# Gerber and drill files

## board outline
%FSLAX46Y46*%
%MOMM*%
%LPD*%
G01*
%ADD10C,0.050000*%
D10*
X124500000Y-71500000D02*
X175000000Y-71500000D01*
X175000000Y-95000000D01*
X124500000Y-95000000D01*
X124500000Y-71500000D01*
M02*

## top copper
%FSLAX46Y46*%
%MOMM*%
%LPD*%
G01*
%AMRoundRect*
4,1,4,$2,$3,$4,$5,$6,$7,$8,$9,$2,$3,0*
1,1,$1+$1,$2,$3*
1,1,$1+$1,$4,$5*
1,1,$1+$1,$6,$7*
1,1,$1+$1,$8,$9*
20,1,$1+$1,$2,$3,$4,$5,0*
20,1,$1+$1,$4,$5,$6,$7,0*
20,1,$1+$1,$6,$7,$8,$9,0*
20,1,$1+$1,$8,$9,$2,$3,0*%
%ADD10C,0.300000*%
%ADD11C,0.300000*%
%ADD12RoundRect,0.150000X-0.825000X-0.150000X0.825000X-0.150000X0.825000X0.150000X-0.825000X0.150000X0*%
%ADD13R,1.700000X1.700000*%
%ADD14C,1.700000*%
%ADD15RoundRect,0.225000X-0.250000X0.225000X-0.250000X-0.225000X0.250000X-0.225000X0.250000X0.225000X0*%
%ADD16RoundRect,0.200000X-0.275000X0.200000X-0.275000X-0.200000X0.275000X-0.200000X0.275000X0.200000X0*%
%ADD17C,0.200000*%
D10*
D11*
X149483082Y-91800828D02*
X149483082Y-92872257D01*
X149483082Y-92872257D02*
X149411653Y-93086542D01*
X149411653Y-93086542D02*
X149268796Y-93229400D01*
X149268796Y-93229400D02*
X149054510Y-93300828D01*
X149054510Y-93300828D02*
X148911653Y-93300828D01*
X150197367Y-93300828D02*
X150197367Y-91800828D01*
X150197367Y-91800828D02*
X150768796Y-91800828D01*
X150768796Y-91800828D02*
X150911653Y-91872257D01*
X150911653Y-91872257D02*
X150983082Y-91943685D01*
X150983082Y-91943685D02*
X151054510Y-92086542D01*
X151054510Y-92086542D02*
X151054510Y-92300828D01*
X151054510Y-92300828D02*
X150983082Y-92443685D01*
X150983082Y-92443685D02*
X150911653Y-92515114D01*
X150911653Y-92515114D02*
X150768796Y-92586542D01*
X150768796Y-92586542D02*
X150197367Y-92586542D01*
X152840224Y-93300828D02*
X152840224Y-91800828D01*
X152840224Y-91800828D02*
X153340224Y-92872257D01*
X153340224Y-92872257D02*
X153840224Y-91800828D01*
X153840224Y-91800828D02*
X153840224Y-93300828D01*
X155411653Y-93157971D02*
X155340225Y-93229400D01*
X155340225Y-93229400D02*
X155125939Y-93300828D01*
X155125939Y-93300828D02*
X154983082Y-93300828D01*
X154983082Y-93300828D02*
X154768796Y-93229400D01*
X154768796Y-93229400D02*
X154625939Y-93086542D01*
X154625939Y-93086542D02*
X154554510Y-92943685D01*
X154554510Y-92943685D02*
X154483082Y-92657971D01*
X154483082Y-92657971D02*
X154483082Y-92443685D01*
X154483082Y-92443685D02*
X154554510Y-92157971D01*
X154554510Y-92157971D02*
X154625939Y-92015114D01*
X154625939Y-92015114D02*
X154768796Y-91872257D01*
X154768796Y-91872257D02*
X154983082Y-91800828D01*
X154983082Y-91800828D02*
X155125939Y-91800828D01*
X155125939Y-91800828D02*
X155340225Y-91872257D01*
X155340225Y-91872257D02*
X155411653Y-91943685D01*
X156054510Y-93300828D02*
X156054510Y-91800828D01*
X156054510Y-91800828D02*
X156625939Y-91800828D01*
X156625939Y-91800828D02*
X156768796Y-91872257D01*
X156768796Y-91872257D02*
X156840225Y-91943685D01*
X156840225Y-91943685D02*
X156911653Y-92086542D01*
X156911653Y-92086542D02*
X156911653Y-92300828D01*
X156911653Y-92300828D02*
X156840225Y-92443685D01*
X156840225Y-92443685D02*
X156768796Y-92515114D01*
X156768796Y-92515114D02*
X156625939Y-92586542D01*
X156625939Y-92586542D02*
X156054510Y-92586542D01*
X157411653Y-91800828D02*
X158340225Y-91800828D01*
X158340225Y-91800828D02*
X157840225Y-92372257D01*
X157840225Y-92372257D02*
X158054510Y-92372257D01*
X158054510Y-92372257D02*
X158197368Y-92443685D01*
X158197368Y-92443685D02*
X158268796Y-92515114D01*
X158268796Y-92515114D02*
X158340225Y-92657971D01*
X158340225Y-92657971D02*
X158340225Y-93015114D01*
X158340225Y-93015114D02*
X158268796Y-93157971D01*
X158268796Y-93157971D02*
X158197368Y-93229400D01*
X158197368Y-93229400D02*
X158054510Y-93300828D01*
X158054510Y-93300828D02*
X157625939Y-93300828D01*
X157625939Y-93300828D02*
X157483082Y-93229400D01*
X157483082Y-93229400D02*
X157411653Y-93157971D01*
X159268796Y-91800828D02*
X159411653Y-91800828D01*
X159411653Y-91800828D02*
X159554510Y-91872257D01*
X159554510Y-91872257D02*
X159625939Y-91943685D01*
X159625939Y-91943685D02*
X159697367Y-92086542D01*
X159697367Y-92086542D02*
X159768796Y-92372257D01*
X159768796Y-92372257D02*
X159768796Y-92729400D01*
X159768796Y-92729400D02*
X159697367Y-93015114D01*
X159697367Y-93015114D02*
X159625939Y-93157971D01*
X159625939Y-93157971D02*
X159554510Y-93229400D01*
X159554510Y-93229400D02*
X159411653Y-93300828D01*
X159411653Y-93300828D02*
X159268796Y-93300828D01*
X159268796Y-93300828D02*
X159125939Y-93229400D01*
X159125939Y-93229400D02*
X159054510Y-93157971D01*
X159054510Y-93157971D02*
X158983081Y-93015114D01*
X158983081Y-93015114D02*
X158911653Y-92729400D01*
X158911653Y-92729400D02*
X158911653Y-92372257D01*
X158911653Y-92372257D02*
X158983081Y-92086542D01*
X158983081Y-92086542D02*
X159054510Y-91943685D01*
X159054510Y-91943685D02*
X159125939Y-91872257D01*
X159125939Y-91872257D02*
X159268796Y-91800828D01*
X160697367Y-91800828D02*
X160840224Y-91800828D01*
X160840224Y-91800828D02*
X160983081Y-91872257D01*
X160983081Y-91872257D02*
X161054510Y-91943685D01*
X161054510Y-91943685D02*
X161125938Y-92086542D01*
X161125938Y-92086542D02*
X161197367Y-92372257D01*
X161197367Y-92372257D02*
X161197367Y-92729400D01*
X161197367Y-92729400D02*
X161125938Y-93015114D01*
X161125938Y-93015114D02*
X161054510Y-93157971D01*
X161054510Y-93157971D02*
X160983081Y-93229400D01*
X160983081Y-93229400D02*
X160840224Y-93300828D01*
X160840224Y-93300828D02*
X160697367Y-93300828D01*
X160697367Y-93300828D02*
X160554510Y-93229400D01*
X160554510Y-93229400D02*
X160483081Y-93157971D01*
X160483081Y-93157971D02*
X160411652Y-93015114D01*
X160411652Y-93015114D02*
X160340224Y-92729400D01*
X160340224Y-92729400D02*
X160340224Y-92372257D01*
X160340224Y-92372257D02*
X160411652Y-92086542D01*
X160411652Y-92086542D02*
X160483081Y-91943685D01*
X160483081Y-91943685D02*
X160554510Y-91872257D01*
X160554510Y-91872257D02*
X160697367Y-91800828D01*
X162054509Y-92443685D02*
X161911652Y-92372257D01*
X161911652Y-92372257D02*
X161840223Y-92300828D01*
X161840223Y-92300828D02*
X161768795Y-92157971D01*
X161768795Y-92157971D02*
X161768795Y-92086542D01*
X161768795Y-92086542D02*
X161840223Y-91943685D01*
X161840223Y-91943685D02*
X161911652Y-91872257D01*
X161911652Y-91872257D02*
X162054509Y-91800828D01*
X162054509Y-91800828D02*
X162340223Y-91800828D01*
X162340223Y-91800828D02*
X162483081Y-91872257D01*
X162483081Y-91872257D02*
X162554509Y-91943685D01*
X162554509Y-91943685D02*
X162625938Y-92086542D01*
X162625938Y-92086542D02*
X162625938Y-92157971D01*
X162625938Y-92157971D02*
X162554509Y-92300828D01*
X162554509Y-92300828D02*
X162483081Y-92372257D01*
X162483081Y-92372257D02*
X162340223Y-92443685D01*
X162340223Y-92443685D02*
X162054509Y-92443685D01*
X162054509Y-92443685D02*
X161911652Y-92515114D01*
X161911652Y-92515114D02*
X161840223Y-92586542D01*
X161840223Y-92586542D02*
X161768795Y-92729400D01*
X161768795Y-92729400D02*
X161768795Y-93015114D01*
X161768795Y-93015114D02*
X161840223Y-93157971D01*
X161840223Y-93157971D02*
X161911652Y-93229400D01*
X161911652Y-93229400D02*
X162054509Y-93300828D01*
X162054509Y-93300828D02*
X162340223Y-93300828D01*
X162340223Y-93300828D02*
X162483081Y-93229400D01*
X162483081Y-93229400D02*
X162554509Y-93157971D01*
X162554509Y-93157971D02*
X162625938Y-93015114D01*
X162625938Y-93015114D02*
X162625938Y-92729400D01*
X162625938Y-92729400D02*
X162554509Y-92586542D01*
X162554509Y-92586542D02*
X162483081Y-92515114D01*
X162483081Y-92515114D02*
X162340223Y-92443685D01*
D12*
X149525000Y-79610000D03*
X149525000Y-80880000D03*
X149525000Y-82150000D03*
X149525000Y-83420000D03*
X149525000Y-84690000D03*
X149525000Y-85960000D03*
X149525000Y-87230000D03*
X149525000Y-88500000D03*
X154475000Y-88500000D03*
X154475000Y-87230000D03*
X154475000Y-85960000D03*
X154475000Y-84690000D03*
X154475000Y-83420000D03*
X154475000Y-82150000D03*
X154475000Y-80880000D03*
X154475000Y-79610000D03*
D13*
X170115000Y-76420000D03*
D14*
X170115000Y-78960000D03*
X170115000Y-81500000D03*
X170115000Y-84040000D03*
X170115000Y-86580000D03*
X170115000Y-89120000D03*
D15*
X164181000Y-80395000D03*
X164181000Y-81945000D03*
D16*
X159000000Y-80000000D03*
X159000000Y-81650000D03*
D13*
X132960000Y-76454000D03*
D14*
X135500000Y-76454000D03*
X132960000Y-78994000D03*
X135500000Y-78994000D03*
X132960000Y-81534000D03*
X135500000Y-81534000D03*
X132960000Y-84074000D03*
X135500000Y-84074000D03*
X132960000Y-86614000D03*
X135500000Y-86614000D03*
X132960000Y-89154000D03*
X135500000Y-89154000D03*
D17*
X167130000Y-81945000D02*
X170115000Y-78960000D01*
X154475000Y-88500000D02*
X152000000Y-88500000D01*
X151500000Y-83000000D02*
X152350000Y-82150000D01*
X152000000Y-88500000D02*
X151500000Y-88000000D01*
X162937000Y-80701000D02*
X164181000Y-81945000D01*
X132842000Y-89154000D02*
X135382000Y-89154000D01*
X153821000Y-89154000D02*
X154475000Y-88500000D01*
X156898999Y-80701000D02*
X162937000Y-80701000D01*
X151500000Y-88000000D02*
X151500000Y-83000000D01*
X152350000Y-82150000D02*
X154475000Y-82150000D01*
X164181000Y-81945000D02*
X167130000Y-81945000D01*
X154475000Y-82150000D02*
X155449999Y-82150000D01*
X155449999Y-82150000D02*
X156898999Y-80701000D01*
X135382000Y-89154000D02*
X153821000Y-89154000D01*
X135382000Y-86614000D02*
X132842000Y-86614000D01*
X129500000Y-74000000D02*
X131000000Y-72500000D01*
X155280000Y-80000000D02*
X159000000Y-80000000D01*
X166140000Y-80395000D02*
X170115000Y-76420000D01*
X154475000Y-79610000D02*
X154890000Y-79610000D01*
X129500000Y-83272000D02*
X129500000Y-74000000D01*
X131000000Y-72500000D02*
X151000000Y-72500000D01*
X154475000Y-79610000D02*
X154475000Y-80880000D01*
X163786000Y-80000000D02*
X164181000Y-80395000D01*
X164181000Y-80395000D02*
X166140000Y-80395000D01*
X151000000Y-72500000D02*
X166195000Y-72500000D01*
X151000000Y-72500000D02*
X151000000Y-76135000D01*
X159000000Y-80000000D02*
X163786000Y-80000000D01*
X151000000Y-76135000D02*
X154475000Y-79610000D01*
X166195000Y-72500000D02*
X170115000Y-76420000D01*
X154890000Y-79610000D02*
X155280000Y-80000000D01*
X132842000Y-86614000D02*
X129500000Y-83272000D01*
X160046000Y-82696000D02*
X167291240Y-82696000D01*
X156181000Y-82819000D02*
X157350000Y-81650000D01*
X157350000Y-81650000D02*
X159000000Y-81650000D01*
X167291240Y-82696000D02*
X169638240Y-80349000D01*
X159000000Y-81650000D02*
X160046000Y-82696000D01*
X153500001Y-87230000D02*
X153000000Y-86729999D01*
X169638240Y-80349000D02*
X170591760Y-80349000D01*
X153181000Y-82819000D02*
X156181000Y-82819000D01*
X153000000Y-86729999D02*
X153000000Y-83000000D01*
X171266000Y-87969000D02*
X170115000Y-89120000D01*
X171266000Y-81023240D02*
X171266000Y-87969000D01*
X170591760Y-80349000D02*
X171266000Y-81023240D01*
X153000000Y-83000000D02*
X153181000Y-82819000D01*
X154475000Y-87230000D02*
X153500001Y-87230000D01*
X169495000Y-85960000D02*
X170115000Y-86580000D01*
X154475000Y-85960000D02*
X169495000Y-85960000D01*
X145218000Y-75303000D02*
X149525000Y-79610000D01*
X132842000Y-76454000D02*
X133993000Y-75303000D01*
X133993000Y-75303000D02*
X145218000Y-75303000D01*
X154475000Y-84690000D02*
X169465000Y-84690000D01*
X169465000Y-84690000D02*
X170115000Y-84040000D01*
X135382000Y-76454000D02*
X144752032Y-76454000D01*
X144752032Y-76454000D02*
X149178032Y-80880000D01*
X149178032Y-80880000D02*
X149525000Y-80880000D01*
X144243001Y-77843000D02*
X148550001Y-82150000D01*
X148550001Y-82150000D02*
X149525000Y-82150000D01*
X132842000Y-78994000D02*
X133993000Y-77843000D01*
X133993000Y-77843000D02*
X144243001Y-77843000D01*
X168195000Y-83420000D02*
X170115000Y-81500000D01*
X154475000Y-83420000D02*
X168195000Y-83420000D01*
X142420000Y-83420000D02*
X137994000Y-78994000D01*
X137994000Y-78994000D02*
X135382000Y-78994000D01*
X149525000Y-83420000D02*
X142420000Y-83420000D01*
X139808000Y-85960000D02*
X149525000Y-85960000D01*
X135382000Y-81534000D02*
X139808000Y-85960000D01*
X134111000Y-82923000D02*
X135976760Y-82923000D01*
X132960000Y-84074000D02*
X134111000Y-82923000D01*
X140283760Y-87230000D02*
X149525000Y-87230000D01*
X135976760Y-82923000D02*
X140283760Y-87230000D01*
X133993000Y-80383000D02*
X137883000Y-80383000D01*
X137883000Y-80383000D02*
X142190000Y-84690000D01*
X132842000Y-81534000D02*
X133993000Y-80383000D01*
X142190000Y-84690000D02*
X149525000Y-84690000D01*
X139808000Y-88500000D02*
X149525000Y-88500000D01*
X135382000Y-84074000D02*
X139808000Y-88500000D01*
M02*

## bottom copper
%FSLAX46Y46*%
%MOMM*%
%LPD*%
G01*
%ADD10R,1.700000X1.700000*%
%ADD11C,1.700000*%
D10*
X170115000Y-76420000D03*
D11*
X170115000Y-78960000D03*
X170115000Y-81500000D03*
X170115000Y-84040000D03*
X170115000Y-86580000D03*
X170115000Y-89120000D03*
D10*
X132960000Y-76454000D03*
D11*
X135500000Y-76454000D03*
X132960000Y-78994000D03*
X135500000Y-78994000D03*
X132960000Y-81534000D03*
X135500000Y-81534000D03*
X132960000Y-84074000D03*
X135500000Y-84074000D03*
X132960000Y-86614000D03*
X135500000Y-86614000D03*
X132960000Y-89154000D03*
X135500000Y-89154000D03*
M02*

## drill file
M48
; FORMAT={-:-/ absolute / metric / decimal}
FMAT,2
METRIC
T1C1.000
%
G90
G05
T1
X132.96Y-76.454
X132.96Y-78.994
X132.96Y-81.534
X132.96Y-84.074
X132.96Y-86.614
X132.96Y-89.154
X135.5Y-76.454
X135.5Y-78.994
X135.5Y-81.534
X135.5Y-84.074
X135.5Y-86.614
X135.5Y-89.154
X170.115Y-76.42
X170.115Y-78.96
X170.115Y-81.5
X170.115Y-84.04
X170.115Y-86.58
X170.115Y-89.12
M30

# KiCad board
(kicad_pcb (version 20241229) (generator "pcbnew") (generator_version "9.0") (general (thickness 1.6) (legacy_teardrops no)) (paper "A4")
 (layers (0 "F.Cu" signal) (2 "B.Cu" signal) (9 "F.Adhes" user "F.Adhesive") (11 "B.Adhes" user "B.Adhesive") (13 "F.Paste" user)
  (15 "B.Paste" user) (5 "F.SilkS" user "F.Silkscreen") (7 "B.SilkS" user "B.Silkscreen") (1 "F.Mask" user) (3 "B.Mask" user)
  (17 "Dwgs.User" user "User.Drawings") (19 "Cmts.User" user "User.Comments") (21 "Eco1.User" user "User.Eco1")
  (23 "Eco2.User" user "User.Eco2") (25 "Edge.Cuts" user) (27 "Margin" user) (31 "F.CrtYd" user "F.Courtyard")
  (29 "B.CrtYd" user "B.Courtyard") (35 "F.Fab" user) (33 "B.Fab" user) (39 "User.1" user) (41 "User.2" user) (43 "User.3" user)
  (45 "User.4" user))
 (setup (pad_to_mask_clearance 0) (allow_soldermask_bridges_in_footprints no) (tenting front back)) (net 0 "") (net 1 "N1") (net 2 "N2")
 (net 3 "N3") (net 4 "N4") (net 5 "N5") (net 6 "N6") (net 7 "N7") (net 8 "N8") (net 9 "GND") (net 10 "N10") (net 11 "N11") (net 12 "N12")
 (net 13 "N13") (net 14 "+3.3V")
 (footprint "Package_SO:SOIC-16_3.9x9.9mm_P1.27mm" (layer "F.Cu") (at 152 84.055)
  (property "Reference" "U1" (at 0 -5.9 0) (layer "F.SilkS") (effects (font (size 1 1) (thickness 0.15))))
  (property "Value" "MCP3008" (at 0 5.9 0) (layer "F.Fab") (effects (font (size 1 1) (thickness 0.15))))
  (pad "1" smd roundrect (at -2.475 -4.445) (size 1.95 0.6) (layers "F.Cu" "F.Mask" "F.Paste") (roundrect_rratio 0.25) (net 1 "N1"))
  (pad "2" smd roundrect (at -2.475 -3.175) (size 1.95 0.6) (layers "F.Cu" "F.Mask" "F.Paste") (roundrect_rratio 0.25) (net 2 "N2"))
  (pad "3" smd roundrect (at -2.475 -1.905) (size 1.95 0.6) (layers "F.Cu" "F.Mask" "F.Paste") (roundrect_rratio 0.25) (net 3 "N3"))
  (pad "4" smd roundrect (at -2.475 -0.635) (size 1.95 0.6) (layers "F.Cu" "F.Mask" "F.Paste") (roundrect_rratio 0.25) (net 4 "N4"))
  (pad "5" smd roundrect (at -2.475 0.635) (size 1.95 0.6) (layers "F.Cu" "F.Mask" "F.Paste") (roundrect_rratio 0.25) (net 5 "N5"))
  (pad "6" smd roundrect (at -2.475 1.905) (size 1.95 0.6) (layers "F.Cu" "F.Mask" "F.Paste") (roundrect_rratio 0.25) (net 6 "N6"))
  (pad "7" smd roundrect (at -2.475 3.175) (size 1.95 0.6) (layers "F.Cu" "F.Mask" "F.Paste") (roundrect_rratio 0.25) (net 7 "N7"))
  (pad "8" smd roundrect (at -2.475 4.445) (size 1.95 0.6) (layers "F.Cu" "F.Mask" "F.Paste") (roundrect_rratio 0.25) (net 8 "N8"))
  (pad "9" smd roundrect (at 2.475 4.445) (size 1.95 0.6) (layers "F.Cu" "F.Mask" "F.Paste") (roundrect_rratio 0.25) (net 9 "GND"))
  (pad "10" smd roundrect (at 2.475 3.175) (size 1.95 0.6) (layers "F.Cu" "F.Mask" "F.Paste") (roundrect_rratio 0.25) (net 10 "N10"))
  (pad "11" smd roundrect (at 2.475 1.905) (size 1.95 0.6) (layers "F.Cu" "F.Mask" "F.Paste") (roundrect_rratio 0.25) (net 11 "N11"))
  (pad "12" smd roundrect (at 2.475 0.635) (size 1.95 0.6) (layers "F.Cu" "F.Mask" "F.Paste") (roundrect_rratio 0.25) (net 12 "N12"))
  (pad "13" smd roundrect (at 2.475 -0.635) (size 1.95 0.6) (layers "F.Cu" "F.Mask" "F.Paste") (roundrect_rratio 0.25) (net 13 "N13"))
  (pad "14" smd roundrect (at 2.475 -1.905) (size 1.95 0.6) (layers "F.Cu" "F.Mask" "F.Paste") (roundrect_rratio 0.25) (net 9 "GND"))
  (pad "15" smd roundrect (at 2.475 -3.175) (size 1.95 0.6) (layers "F.Cu" "F.Mask" "F.Paste") (roundrect_rratio 0.25) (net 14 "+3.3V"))
  (pad "16" smd roundrect (at 2.475 -4.445) (size 1.95 0.6) (layers "F.Cu" "F.Mask" "F.Paste") (roundrect_rratio 0.25) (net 14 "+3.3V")))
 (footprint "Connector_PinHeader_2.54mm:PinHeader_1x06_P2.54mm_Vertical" (layer "F.Cu") (at 170.115 76.42)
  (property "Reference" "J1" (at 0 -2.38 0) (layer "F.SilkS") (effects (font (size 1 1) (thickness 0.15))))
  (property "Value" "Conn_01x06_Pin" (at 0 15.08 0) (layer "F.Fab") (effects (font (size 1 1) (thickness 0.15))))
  (pad "1" thru_hole rect (at 0 0) (size 1.7 1.7) (drill 1) (layers "*.Cu" "*.Mask") (remove_unused_layers no) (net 14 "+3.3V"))
  (pad "2" thru_hole circle (at 0 2.54) (size 1.7 1.7) (drill 1) (layers "*.Cu" "*.Mask") (remove_unused_layers no) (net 9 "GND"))
  (pad "3" thru_hole circle (at 0 5.08) (size 1.7 1.7) (drill 1) (layers "*.Cu" "*.Mask") (remove_unused_layers no) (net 13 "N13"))
  (pad "4" thru_hole circle (at 0 7.62) (size 1.7 1.7) (drill 1) (layers "*.Cu" "*.Mask") (remove_unused_layers no) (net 12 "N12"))
  (pad "5" thru_hole circle (at 0 10.16) (size 1.7 1.7) (drill 1) (layers "*.Cu" "*.Mask") (remove_unused_layers no) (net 11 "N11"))
  (pad "6" thru_hole circle (at 0 12.7) (size 1.7 1.7) (drill 1) (layers "*.Cu" "*.Mask") (remove_unused_layers no) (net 10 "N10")))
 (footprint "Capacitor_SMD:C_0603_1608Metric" (layer "F.Cu") (at 164.181 81.17 -90)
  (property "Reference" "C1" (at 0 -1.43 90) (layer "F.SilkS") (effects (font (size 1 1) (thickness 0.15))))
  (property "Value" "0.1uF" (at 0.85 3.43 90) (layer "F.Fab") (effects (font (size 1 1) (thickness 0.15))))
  (pad "1" smd roundrect (at -0.775 0 270) (size 0.9 0.95) (layers "F.Cu" "F.Mask" "F.Paste") (roundrect_rratio 0.25) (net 14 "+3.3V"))
  (pad "2" smd roundrect (at 0.775 0 270) (size 0.9 0.95) (layers "F.Cu" "F.Mask" "F.Paste") (roundrect_rratio 0.25) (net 9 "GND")))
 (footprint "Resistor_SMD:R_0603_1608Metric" (layer "F.Cu") (at 159 80.825 -90)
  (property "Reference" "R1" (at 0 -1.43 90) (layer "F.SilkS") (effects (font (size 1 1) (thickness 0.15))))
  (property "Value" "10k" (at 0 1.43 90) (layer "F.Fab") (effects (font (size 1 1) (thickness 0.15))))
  (pad "1" smd roundrect (at -0.825 0 270) (size 0.8 0.95) (layers "F.Cu" "F.Mask" "F.Paste") (roundrect_rratio 0.25) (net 14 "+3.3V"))
  (pad "2" smd roundrect (at 0.825 0 270) (size 0.8 0.95) (layers "F.Cu" "F.Mask" "F.Paste") (roundrect_rratio 0.25) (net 10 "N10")))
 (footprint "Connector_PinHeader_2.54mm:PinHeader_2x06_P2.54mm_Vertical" (layer "F.Cu") (at 132.96 76.454)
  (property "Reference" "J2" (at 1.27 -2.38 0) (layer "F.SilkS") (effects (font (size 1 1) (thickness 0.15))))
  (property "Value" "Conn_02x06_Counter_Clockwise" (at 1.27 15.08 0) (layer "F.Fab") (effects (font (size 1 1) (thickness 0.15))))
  (pad "1" thru_hole rect (at 0 0) (size 1.7 1.7) (drill 1) (layers "*.Cu" "*.Mask") (remove_unused_layers no) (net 1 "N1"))
  (pad "2" thru_hole circle (at 2.54 0) (size 1.7 1.7) (drill 1) (layers "*.Cu" "*.Mask") (remove_unused_layers no) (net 2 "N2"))
  (pad "3" thru_hole circle (at 0 2.54) (size 1.7 1.7) (drill 1) (layers "*.Cu" "*.Mask") (remove_unused_layers no) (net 3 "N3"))
  (pad "4" thru_hole circle (at 2.54 2.54) (size 1.7 1.7) (drill 1) (layers "*.Cu" "*.Mask") (remove_unused_layers no) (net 4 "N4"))
  (pad "5" thru_hole circle (at 0 5.08) (size 1.7 1.7) (drill 1) (layers "*.Cu" "*.Mask") (remove_unused_layers no) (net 5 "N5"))
  (pad "6" thru_hole circle (at 2.54 5.08) (size 1.7 1.7) (drill 1) (layers "*.Cu" "*.Mask") (remove_unused_layers no) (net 6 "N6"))
  (pad "7" thru_hole circle (at 0 7.62) (size 1.7 1.7) (drill 1) (layers "*.Cu" "*.Mask") (remove_unused_layers no) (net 7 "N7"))
  (pad "8" thru_hole circle (at 2.54 7.62) (size 1.7 1.7) (drill 1) (layers "*.Cu" "*.Mask") (remove_unused_layers no) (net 8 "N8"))
  (pad "9" thru_hole circle (at 0 10.16) (size 1.7 1.7) (drill 1) (layers "*.Cu" "*.Mask") (remove_unused_layers no) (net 14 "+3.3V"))
  (pad "10" thru_hole circle (at 2.54 10.16) (size 1.7 1.7) (drill 1) (layers "*.Cu" "*.Mask") (remove_unused_layers no) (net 14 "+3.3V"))
  (pad "11" thru_hole circle (at 0 12.7) (size 1.7 1.7) (drill 1) (layers "*.Cu" "*.Mask") (remove_unused_layers no) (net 9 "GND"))
  (pad "12" thru_hole circle (at 2.54 12.7) (size 1.7 1.7) (drill 1) (layers "*.Cu" "*.Mask") (remove_unused_layers no) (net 9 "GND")))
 (gr_rect (start 124.5 71.5) (end 175 95) (stroke (width 0.05) (type solid)) (fill no) (layer "Edge.Cuts"))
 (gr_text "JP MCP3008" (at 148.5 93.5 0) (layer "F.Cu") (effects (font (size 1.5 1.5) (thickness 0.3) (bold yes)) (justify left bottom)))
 (segment (start 167.13 81.945) (end 170.115 78.96) (width 0.2) (layer "F.Cu") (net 9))
 (segment (start 154.475 88.5) (end 152 88.5) (width 0.2) (layer "F.Cu") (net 9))
 (segment (start 151.5 83) (end 152.35 82.15) (width 0.2) (layer "F.Cu") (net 9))
 (segment (start 152 88.5) (end 151.5 88) (width 0.2) (layer "F.Cu") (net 9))
 (segment (start 162.937 80.701) (end 164.181 81.945) (width 0.2) (layer "F.Cu") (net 9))
 (segment (start 132.842 89.154) (end 135.382 89.154) (width 0.2) (layer "F.Cu") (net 9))
 (segment (start 153.821 89.154) (end 154.475 88.5) (width 0.2) (layer "F.Cu") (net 9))
 (segment (start 156.898999 80.701) (end 162.937 80.701) (width 0.2) (layer "F.Cu") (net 9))
 (segment (start 151.5 88) (end 151.5 83) (width 0.2) (layer "F.Cu") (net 9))
 (segment (start 152.35 82.15) (end 154.475 82.15) (width 0.2) (layer "F.Cu") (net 9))
 (segment (start 164.181 81.945) (end 167.13 81.945) (width 0.2) (layer "F.Cu") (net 9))
 (segment (start 154.475 82.15) (end 155.449999 82.15) (width 0.2) (layer "F.Cu") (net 9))
 (segment (start 155.449999 82.15) (end 156.898999 80.701) (width 0.2) (layer "F.Cu") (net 9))
 (segment (start 135.382 89.154) (end 153.821 89.154) (width 0.2) (layer "F.Cu") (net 9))
 (segment (start 135.382 86.614) (end 132.842 86.614) (width 0.2) (layer "F.Cu") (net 14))
 (segment (start 129.5 74) (end 131 72.5) (width 0.2) (layer "F.Cu") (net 14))
 (segment (start 155.28 80) (end 159 80) (width 0.2) (layer "F.Cu") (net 14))
 (segment (start 166.14 80.395) (end 170.115 76.42) (width 0.2) (layer "F.Cu") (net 14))
 (segment (start 154.475 79.61) (end 154.89 79.61) (width 0.2) (layer "F.Cu") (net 14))
 (segment (start 129.5 83.272) (end 129.5 74) (width 0.2) (layer "F.Cu") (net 14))
 (segment (start 131 72.5) (end 151 72.5) (width 0.2) (layer "F.Cu") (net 14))
 (segment (start 154.475 79.61) (end 154.475 80.88) (width 0.2) (layer "F.Cu") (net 14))
 (segment (start 163.786 80) (end 164.181 80.395) (width 0.2) (layer "F.Cu") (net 14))
 (segment (start 164.181 80.395) (end 166.14 80.395) (width 0.2) (layer "F.Cu") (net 14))
 (segment (start 151 72.5) (end 166.195 72.5) (width 0.2) (layer "F.Cu") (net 14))
 (segment (start 151 72.5) (end 151 76.135) (width 0.2) (layer "F.Cu") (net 14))
 (segment (start 159 80) (end 163.786 80) (width 0.2) (layer "F.Cu") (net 14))
 (segment (start 151 76.135) (end 154.475 79.61) (width 0.2) (layer "F.Cu") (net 14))
 (segment (start 166.195 72.5) (end 170.115 76.42) (width 0.2) (layer "F.Cu") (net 14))
 (segment (start 154.89 79.61) (end 155.28 80) (width 0.2) (layer "F.Cu") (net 14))
 (segment (start 132.842 86.614) (end 129.5 83.272) (width 0.2) (layer "F.Cu") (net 14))
 (segment (start 160.046 82.696) (end 167.29124 82.696) (width 0.2) (layer "F.Cu") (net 10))
 (segment (start 156.181 82.819) (end 157.35 81.65) (width 0.2) (layer "F.Cu") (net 10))
 (segment (start 157.35 81.65) (end 159 81.65) (width 0.2) (layer "F.Cu") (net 10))
 (segment (start 167.29124 82.696) (end 169.63824 80.349) (width 0.2) (layer "F.Cu") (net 10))
 (segment (start 159 81.65) (end 160.046 82.696) (width 0.2) (layer "F.Cu") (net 10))
 (segment (start 153.500001 87.23) (end 153 86.729999) (width 0.2) (layer "F.Cu") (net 10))
 (segment (start 169.63824 80.349) (end 170.59176 80.349) (width 0.2) (layer "F.Cu") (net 10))
 (segment (start 153.181 82.819) (end 156.181 82.819) (width 0.2) (layer "F.Cu") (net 10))
 (segment (start 153 86.729999) (end 153 83) (width 0.2) (layer "F.Cu") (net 10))
 (segment (start 171.266 87.969) (end 170.115 89.12) (width 0.2) (layer "F.Cu") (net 10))
 (segment (start 171.266 81.02324) (end 171.266 87.969) (width 0.2) (layer "F.Cu") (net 10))
 (segment (start 170.59176 80.349) (end 171.266 81.02324) (width 0.2) (layer "F.Cu") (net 10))
 (segment (start 153 83) (end 153.181 82.819) (width 0.2) (layer "F.Cu") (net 10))
 (segment (start 154.475 87.23) (end 153.500001 87.23) (width 0.2) (layer "F.Cu") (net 10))
 (segment (start 169.495 85.96) (end 170.115 86.58) (width 0.2) (layer "F.Cu") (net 11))
 (segment (start 154.475 85.96) (end 169.495 85.96) (width 0.2) (layer "F.Cu") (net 11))
 (segment (start 145.218 75.303) (end 149.525 79.61) (width 0.2) (layer "F.Cu") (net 1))
 (segment (start 132.842 76.454) (end 133.993 75.303) (width 0.2) (layer "F.Cu") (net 1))
 (segment (start 133.993 75.303) (end 145.218 75.303) (width 0.2) (layer "F.Cu") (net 1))
 (segment (start 154.475 84.69) (end 169.465 84.69) (width 0.2) (layer "F.Cu") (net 12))
 (segment (start 169.465 84.69) (end 170.115 84.04) (width 0.2) (layer "F.Cu") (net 12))
 (segment (start 135.382 76.454) (end 144.752032 76.454) (width 0.2) (layer "F.Cu") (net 2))
 (segment (start 144.752032 76.454) (end 149.178032 80.88) (width 0.2) (layer "F.Cu") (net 2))
 (segment (start 149.178032 80.88) (end 149.525 80.88) (width 0.2) (layer "F.Cu") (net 2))
 (segment (start 144.243001 77.843) (end 148.550001 82.15) (width 0.2) (layer "F.Cu") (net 3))
 (segment (start 148.550001 82.15) (end 149.525 82.15) (width 0.2) (layer "F.Cu") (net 3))
 (segment (start 132.842 78.994) (end 133.993 77.843) (width 0.2) (layer "F.Cu") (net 3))
 (segment (start 133.993 77.843) (end 144.243001 77.843) (width 0.2) (layer "F.Cu") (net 3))
 (segment (start 168.195 83.42) (end 170.115 81.5) (width 0.2) (layer "F.Cu") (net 13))
 (segment (start 154.475 83.42) (end 168.195 83.42) (width 0.2) (layer "F.Cu") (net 13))
 (segment (start 142.42 83.42) (end 137.994 78.994) (width 0.2) (layer "F.Cu") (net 4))
 (segment (start 137.994 78.994) (end 135.382 78.994) (width 0.2) (layer "F.Cu") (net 4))
 (segment (start 149.525 83.42) (end 142.42 83.42) (width 0.2) (layer "F.Cu") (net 4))
 (segment (start 139.808 85.96) (end 149.525 85.96) (width 0.2) (layer "F.Cu") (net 6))
 (segment (start 135.382 81.534) (end 139.808 85.96) (width 0.2) (layer "F.Cu") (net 6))
 (segment (start 134.111 82.923) (end 135.97676 82.923) (width 0.2) (layer "F.Cu") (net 7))
 (segment (start 132.96 84.074) (end 134.111 82.923) (width 0.2) (layer "F.Cu") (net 7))
 (segment (start 140.28376 87.23) (end 149.525 87.23) (width 0.2) (layer "F.Cu") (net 7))
 (segment (start 135.97676 82.923) (end 140.28376 87.23) (width 0.2) (layer "F.Cu") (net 7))
 (segment (start 133.993 80.383) (end 137.883 80.383) (width 0.2) (layer "F.Cu") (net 5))
 (segment (start 137.883 80.383) (end 142.19 84.69) (width 0.2) (layer "F.Cu") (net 5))
 (segment (start 132.842 81.534) (end 133.993 80.383) (width 0.2) (layer "F.Cu") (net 5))
 (segment (start 142.19 84.69) (end 149.525 84.69) (width 0.2) (layer "F.Cu") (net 5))
 (segment (start 139.808 88.5) (end 149.525 88.5) (width 0.2) (layer "F.Cu") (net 8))
 (segment (start 135.382 84.074) (end 139.808 88.5) (width 0.2) (layer "F.Cu") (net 8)))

